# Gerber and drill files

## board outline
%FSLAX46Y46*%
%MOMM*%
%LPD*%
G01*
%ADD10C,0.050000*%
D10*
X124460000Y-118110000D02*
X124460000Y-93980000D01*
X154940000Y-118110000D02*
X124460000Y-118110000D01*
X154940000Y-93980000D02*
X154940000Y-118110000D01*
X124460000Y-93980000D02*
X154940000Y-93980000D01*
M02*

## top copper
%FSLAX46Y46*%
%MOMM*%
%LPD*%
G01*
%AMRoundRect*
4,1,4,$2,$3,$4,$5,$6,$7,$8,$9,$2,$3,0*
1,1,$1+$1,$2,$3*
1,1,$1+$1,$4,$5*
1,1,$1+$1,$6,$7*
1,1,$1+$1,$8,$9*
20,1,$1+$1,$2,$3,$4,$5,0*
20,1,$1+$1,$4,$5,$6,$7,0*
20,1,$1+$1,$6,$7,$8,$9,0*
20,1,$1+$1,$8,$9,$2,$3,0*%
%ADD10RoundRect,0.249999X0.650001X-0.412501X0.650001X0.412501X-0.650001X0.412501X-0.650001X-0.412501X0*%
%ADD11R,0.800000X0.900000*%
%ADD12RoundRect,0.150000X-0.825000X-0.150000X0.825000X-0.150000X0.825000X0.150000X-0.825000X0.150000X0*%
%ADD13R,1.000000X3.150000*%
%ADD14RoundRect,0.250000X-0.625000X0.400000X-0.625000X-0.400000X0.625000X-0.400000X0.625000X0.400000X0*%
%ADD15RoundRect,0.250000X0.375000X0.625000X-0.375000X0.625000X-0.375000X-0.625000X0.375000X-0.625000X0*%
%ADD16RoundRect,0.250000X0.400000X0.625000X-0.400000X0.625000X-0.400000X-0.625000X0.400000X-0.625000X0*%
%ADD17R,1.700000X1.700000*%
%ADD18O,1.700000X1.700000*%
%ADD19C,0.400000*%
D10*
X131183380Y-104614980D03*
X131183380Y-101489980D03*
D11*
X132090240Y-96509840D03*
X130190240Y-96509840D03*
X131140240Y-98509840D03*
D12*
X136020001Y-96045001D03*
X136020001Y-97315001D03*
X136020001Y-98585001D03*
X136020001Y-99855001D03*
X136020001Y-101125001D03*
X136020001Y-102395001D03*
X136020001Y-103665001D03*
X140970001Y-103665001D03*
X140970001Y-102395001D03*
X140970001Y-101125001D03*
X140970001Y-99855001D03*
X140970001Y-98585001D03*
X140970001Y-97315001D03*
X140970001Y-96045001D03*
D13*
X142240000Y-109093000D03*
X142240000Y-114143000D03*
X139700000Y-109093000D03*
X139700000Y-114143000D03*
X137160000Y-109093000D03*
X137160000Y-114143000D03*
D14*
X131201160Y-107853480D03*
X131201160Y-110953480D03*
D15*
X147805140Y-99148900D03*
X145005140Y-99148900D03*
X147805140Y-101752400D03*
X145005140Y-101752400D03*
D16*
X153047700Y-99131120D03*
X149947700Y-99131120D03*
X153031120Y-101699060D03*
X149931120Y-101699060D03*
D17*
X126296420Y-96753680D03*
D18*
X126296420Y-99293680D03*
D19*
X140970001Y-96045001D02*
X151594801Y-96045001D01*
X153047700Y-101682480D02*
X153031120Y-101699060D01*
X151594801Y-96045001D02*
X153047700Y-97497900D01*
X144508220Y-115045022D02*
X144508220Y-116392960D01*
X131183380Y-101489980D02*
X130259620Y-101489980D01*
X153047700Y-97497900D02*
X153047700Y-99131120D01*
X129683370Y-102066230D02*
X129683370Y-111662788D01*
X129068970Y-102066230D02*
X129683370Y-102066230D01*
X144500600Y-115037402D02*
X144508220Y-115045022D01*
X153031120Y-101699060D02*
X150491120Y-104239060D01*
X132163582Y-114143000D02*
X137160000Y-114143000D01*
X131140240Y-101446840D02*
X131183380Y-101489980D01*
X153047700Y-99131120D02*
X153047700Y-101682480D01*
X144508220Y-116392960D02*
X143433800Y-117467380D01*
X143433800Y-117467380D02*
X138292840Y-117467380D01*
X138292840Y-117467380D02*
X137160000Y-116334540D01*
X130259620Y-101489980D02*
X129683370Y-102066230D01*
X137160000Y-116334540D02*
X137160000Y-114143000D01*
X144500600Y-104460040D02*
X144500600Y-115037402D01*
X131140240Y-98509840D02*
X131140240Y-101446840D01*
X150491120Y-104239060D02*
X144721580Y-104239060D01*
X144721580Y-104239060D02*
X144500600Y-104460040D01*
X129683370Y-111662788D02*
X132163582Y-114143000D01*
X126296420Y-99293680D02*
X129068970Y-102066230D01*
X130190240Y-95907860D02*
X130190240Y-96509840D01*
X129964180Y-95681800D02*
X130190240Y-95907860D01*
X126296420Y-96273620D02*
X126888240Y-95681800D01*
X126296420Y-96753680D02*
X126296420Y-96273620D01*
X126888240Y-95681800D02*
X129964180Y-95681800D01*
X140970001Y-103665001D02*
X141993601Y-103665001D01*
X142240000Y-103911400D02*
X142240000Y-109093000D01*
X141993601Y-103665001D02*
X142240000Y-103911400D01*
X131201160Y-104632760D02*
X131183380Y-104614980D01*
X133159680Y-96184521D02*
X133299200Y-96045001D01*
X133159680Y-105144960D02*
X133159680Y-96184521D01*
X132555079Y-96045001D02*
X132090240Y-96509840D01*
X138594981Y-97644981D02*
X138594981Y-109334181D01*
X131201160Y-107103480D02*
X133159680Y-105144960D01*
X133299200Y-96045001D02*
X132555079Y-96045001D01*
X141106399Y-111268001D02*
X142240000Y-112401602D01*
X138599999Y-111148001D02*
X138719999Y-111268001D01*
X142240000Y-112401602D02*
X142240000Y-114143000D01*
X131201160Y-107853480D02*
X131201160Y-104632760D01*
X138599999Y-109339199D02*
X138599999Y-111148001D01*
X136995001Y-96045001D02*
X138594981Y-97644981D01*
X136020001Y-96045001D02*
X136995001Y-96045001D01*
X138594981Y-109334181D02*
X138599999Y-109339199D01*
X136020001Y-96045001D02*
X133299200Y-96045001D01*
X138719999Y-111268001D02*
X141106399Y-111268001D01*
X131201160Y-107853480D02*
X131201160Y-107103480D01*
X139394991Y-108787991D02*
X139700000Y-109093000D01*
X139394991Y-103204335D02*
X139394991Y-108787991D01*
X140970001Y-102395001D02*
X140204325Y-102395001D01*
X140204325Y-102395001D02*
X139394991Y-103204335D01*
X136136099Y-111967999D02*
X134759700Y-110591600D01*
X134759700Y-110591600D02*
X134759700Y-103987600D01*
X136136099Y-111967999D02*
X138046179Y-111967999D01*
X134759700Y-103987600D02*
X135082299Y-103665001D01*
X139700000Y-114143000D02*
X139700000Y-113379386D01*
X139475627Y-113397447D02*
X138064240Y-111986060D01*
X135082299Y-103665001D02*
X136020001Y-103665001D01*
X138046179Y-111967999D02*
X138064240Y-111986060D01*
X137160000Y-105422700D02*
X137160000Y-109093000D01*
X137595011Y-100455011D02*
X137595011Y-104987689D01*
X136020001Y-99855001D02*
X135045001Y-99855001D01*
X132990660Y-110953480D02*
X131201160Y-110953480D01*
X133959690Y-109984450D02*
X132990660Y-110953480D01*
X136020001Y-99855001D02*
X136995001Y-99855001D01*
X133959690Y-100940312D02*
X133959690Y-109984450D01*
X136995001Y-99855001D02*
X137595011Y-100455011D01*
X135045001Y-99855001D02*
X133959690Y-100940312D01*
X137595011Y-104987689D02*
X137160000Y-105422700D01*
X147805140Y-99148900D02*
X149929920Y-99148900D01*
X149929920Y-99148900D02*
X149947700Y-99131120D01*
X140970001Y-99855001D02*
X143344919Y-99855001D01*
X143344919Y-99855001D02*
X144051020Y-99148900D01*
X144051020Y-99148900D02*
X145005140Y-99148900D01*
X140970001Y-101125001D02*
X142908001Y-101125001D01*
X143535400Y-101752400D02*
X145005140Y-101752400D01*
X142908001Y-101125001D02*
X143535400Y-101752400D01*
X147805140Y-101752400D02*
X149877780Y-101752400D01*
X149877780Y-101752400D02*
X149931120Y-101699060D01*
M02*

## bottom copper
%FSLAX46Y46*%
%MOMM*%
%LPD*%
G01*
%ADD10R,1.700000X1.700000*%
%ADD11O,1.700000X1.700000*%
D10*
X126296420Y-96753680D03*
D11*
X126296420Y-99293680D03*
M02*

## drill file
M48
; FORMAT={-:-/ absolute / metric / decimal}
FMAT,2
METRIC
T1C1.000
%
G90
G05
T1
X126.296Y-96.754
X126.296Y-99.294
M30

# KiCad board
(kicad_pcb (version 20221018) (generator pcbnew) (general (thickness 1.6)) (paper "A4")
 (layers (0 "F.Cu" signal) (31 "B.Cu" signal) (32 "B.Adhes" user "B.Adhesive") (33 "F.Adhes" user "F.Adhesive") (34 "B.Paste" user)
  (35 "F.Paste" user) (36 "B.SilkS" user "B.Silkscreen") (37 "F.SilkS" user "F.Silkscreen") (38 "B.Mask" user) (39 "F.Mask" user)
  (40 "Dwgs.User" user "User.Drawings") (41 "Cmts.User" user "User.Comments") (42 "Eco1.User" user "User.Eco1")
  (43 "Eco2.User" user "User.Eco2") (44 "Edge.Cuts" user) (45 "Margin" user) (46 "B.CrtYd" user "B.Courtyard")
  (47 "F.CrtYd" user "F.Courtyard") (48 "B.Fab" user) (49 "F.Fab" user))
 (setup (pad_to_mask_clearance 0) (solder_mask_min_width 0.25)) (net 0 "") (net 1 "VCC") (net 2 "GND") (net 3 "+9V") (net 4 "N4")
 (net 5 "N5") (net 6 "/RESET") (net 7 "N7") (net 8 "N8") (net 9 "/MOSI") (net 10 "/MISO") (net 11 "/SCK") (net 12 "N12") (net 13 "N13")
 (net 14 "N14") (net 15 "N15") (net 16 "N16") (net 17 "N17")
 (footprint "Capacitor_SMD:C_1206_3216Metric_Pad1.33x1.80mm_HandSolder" (layer "F.Cu") (at 131.18338 103.05248 90)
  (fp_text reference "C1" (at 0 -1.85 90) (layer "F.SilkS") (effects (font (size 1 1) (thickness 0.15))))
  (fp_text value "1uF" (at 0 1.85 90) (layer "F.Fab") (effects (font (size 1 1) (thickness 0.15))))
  (pad "1" smd roundrect (at -1.5625 0 90) (size 1.325 1.8) (layers "F.Cu" "F.Paste" "F.Mask") (roundrect_rratio 0.1886784906) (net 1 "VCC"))
  (pad "2" smd roundrect (at 1.5625 0 90) (size 1.325 1.8) (layers "F.Cu" "F.Paste" "F.Mask") (roundrect_rratio 0.1886784906) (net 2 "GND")))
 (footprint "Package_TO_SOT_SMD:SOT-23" (layer "F.Cu") (at 131.14024 97.50984 -90)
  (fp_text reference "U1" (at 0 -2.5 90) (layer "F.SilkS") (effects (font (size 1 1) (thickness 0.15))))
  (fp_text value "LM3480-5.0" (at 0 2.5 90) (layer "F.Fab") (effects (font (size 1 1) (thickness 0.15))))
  (pad "1" smd rect (at -1 -0.95 270) (size 0.9 0.8) (layers "F.Cu" "F.Paste" "F.Mask") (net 1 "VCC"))
  (pad "2" smd rect (at -1 0.95 270) (size 0.9 0.8) (layers "F.Cu" "F.Paste" "F.Mask") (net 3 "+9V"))
  (pad "3" smd rect (at 1 0 270) (size 0.9 0.8) (layers "F.Cu" "F.Paste" "F.Mask") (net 2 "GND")))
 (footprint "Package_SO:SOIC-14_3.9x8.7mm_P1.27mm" (layer "F.Cu") (at 138.495001 99.855001)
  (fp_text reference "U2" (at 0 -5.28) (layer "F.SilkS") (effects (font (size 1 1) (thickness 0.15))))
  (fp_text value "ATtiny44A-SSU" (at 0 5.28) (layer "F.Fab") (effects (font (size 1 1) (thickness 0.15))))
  (pad "1" smd roundrect (at -2.475 -3.81) (size 1.95 0.6) (layers "F.Cu" "F.Paste" "F.Mask") (roundrect_rratio 0.25) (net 1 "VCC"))
  (pad "2" smd roundrect (at -2.475 -2.54) (size 1.95 0.6) (layers "F.Cu" "F.Paste" "F.Mask") (roundrect_rratio 0.25) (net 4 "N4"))
  (pad "3" smd roundrect (at -2.475 -1.27) (size 1.95 0.6) (layers "F.Cu" "F.Paste" "F.Mask") (roundrect_rratio 0.25) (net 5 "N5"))
  (pad "4" smd roundrect (at -2.475 0) (size 1.95 0.6) (layers "F.Cu" "F.Paste" "F.Mask") (roundrect_rratio 0.25) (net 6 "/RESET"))
  (pad "5" smd roundrect (at -2.475 1.27) (size 1.95 0.6) (layers "F.Cu" "F.Paste" "F.Mask") (roundrect_rratio 0.25) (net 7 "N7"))
  (pad "6" smd roundrect (at -2.475 2.54) (size 1.95 0.6) (layers "F.Cu" "F.Paste" "F.Mask") (roundrect_rratio 0.25) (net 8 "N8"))
  (pad "7" smd roundrect (at -2.475 3.81) (size 1.95 0.6) (layers "F.Cu" "F.Paste" "F.Mask") (roundrect_rratio 0.25) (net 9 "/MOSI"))
  (pad "8" smd roundrect (at 2.475 3.81) (size 1.95 0.6) (layers "F.Cu" "F.Paste" "F.Mask") (roundrect_rratio 0.25) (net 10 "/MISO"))
  (pad "9" smd roundrect (at 2.475 2.54) (size 1.95 0.6) (layers "F.Cu" "F.Paste" "F.Mask") (roundrect_rratio 0.25) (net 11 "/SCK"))
  (pad "10" smd roundrect (at 2.475 1.27) (size 1.95 0.6) (layers "F.Cu" "F.Paste" "F.Mask") (roundrect_rratio 0.25) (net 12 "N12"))
  (pad "11" smd roundrect (at 2.475 0) (size 1.95 0.6) (layers "F.Cu" "F.Paste" "F.Mask") (roundrect_rratio 0.25) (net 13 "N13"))
  (pad "12" smd roundrect (at 2.475 -1.27) (size 1.95 0.6) (layers "F.Cu" "F.Paste" "F.Mask") (roundrect_rratio 0.25) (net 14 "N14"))
  (pad "13" smd roundrect (at 2.475 -2.54) (size 1.95 0.6) (layers "F.Cu" "F.Paste" "F.Mask") (roundrect_rratio 0.25) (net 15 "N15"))
  (pad "14" smd roundrect (at 2.475 -3.81) (size 1.95 0.6) (layers "F.Cu" "F.Paste" "F.Mask") (roundrect_rratio 0.25) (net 2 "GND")))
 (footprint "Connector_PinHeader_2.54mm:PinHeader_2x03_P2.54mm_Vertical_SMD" (layer "F.Cu") (at 139.7 111.618 -90)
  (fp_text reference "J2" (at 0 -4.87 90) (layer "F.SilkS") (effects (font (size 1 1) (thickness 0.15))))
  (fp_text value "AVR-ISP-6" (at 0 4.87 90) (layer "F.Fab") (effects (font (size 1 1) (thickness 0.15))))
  (pad "1" smd rect (at -2.525 -2.54 270) (size 3.15 1) (layers "F.Cu" "F.Paste" "F.Mask") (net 10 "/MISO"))
  (pad "2" smd rect (at 2.525 -2.54 270) (size 3.15 1) (layers "F.Cu" "F.Paste" "F.Mask") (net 1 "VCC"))
  (pad "3" smd rect (at -2.525 0 270) (size 3.15 1) (layers "F.Cu" "F.Paste" "F.Mask") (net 11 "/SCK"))
  (pad "4" smd rect (at 2.525 0 270) (size 3.15 1) (layers "F.Cu" "F.Paste" "F.Mask") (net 9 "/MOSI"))
  (pad "5" smd rect (at -2.525 2.54 270) (size 3.15 1) (layers "F.Cu" "F.Paste" "F.Mask") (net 6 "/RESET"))
  (pad "6" smd rect (at 2.525 2.54 270) (size 3.15 1) (layers "F.Cu" "F.Paste" "F.Mask") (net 2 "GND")))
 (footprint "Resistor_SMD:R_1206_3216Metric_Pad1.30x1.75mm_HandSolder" (layer "F.Cu") (at 131.20116 109.40348 -90)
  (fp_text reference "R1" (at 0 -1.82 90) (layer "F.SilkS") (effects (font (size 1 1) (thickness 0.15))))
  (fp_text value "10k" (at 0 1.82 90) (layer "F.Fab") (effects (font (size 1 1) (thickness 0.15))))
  (pad "1" smd roundrect (at -1.55 0 270) (size 1.3 1.75) (layers "F.Cu" "F.Paste" "F.Mask") (roundrect_rratio 0.1923076923) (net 1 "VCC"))
  (pad "2" smd roundrect (at 1.55 0 270) (size 1.3 1.75) (layers "F.Cu" "F.Paste" "F.Mask") (roundrect_rratio 0.1923076923) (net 6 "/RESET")))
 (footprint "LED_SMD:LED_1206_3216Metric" (layer "F.Cu") (at 146.40514 99.1489 180)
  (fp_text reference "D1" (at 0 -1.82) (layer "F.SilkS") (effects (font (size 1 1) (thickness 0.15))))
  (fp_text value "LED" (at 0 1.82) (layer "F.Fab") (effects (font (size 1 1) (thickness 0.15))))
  (pad "1" smd roundrect (at -1.4 0 180) (size 1.25 1.75) (layers "F.Cu" "F.Paste" "F.Mask") (roundrect_rratio 0.2) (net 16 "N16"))
  (pad "2" smd roundrect (at 1.4 0 180) (size 1.25 1.75) (layers "F.Cu" "F.Paste" "F.Mask") (roundrect_rratio 0.2) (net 13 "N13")))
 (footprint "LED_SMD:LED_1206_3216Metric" (layer "F.Cu") (at 146.40514 101.7524 180)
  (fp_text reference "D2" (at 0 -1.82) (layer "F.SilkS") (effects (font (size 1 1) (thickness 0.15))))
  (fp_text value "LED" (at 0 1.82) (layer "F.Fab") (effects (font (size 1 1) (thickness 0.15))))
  (pad "1" smd roundrect (at -1.4 0 180) (size 1.25 1.75) (layers "F.Cu" "F.Paste" "F.Mask") (roundrect_rratio 0.2) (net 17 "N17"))
  (pad "2" smd roundrect (at 1.4 0 180) (size 1.25 1.75) (layers "F.Cu" "F.Paste" "F.Mask") (roundrect_rratio 0.2) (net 12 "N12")))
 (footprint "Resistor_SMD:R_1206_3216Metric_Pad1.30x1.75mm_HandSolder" (layer "F.Cu") (at 151.4977 99.13112 180)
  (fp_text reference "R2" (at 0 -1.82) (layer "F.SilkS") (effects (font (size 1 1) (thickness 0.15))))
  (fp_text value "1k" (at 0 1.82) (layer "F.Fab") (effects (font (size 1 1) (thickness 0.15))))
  (pad "1" smd roundrect (at -1.55 0 180) (size 1.3 1.75) (layers "F.Cu" "F.Paste" "F.Mask") (roundrect_rratio 0.1923076923) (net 2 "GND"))
  (pad "2" smd roundrect (at 1.55 0 180) (size 1.3 1.75) (layers "F.Cu" "F.Paste" "F.Mask") (roundrect_rratio 0.1923076923) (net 16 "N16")))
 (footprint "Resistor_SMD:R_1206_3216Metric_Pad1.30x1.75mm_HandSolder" (layer "F.Cu") (at 151.48112 101.69906 180)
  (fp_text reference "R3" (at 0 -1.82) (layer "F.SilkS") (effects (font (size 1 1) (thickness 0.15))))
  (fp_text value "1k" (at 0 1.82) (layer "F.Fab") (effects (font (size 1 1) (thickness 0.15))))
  (pad "1" smd roundrect (at -1.55 0 180) (size 1.3 1.75) (layers "F.Cu" "F.Paste" "F.Mask") (roundrect_rratio 0.1923076923) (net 2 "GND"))
  (pad "2" smd roundrect (at 1.55 0 180) (size 1.3 1.75) (layers "F.Cu" "F.Paste" "F.Mask") (roundrect_rratio 0.1923076923) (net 17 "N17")))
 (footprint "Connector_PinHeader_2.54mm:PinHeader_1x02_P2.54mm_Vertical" (layer "F.Cu") (at 126.29642 96.75368)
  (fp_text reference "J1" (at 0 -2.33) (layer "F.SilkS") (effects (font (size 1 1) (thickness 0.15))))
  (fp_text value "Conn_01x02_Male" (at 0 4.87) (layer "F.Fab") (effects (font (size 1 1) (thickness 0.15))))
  (pad "1" thru_hole rect (at 0 0) (size 1.7 1.7) (drill 1) (layers "*.Cu" "*.Mask") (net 3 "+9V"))
  (pad "2" thru_hole oval (at 0 2.54) (size 1.7 1.7) (drill 1) (layers "*.Cu" "*.Mask") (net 2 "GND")))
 (gr_line (start 124.46 118.11) (end 124.46 93.98) (stroke (width 0.05) (type solid)) (layer "Edge.Cuts"))
 (gr_line (start 154.94 118.11) (end 124.46 118.11) (stroke (width 0.05) (type solid)) (layer "Edge.Cuts"))
 (gr_line (start 154.94 93.98) (end 154.94 118.11) (stroke (width 0.05) (type solid)) (layer "Edge.Cuts"))
 (gr_line (start 124.46 93.98) (end 154.94 93.98) (stroke (width 0.05) (type solid)) (layer "Edge.Cuts"))
 (segment (start 140.970001 96.045001) (end 151.594801 96.045001) (width 0.4) (layer "F.Cu") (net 2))
 (segment (start 153.0477 101.68248) (end 153.03112 101.69906) (width 0.4) (layer "F.Cu") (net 2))
 (segment (start 151.594801 96.045001) (end 153.0477 97.4979) (width 0.4) (layer "F.Cu") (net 2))
 (segment (start 144.50822 115.045022) (end 144.50822 116.39296) (width 0.4) (layer "F.Cu") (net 2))
 (segment (start 131.18338 101.48998) (end 130.25962 101.48998) (width 0.4) (layer "F.Cu") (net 2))
 (segment (start 153.0477 97.4979) (end 153.0477 99.13112) (width 0.4) (layer "F.Cu") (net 2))
 (segment (start 129.68337 102.06623) (end 129.68337 111.662788) (width 0.4) (layer "F.Cu") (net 2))
 (segment (start 129.06897 102.06623) (end 129.68337 102.06623) (width 0.4) (layer "F.Cu") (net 2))
 (segment (start 144.5006 115.037402) (end 144.50822 115.045022) (width 0.4) (layer "F.Cu") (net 2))
 (segment (start 153.03112 101.69906) (end 150.49112 104.23906) (width 0.4) (layer "F.Cu") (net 2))
 (segment (start 132.163582 114.143) (end 137.16 114.143) (width 0.4) (layer "F.Cu") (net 2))
 (segment (start 131.14024 101.44684) (end 131.18338 101.48998) (width 0.4) (layer "F.Cu") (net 2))
 (segment (start 153.0477 99.13112) (end 153.0477 101.68248) (width 0.4) (layer "F.Cu") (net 2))
 (segment (start 144.50822 116.39296) (end 143.4338 117.46738) (width 0.4) (layer "F.Cu") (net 2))
 (segment (start 143.4338 117.46738) (end 138.29284 117.46738) (width 0.4) (layer "F.Cu") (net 2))
 (segment (start 138.29284 117.46738) (end 137.16 116.33454) (width 0.4) (layer "F.Cu") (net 2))
 (segment (start 130.25962 101.48998) (end 129.68337 102.06623) (width 0.4) (layer "F.Cu") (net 2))
 (segment (start 137.16 116.33454) (end 137.16 114.143) (width 0.4) (layer "F.Cu") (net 2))
 (segment (start 144.5006 104.46004) (end 144.5006 115.037402) (width 0.4) (layer "F.Cu") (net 2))
 (segment (start 131.14024 98.50984) (end 131.14024 101.44684) (width 0.4) (layer "F.Cu") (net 2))
 (segment (start 150.49112 104.23906) (end 144.72158 104.23906) (width 0.4) (layer "F.Cu") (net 2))
 (segment (start 144.72158 104.23906) (end 144.5006 104.46004) (width 0.4) (layer "F.Cu") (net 2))
 (segment (start 129.68337 111.662788) (end 132.163582 114.143) (width 0.4) (layer "F.Cu") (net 2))
 (segment (start 126.29642 99.29368) (end 129.06897 102.06623) (width 0.4) (layer "F.Cu") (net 2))
 (segment (start 130.19024 95.90786) (end 130.19024 96.50984) (width 0.4) (layer "F.Cu") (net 3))
 (segment (start 129.96418 95.6818) (end 130.19024 95.90786) (width 0.4) (layer "F.Cu") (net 3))
 (segment (start 126.29642 96.27362) (end 126.88824 95.6818) (width 0.4) (layer "F.Cu") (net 3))
 (segment (start 126.29642 96.75368) (end 126.29642 96.27362) (width 0.4) (layer "F.Cu") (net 3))
 (segment (start 126.88824 95.6818) (end 129.96418 95.6818) (width 0.4) (layer "F.Cu") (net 3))
 (segment (start 140.970001 103.665001) (end 141.993601 103.665001) (width 0.4) (layer "F.Cu") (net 10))
 (segment (start 142.24 103.9114) (end 142.24 109.093) (width 0.4) (layer "F.Cu") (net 10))
 (segment (start 141.993601 103.665001) (end 142.24 103.9114) (width 0.4) (layer "F.Cu") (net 10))
 (segment (start 131.20116 104.63276) (end 131.18338 104.61498) (width 0.4) (layer "F.Cu") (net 1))
 (segment (start 133.15968 96.184521) (end 133.2992 96.045001) (width 0.4) (layer "F.Cu") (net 1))
 (segment (start 133.15968 105.14496) (end 133.15968 96.184521) (width 0.4) (layer "F.Cu") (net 1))
 (segment (start 132.555079 96.045001) (end 132.09024 96.50984) (width 0.4) (layer "F.Cu") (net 1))
 (segment (start 138.594981 97.644981) (end 138.594981 109.334181) (width 0.4) (layer "F.Cu") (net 1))
 (segment (start 131.20116 107.10348) (end 133.15968 105.14496) (width 0.4) (layer "F.Cu") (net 1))
 (segment (start 133.2992 96.045001) (end 132.555079 96.045001) (width 0.4) (layer "F.Cu") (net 1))
 (segment (start 141.106399 111.268001) (end 142.24 112.401602) (width 0.4) (layer "F.Cu") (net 1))
 (segment (start 138.599999 111.148001) (end 138.719999 111.268001) (width 0.4) (layer "F.Cu") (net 1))
 (segment (start 142.24 112.401602) (end 142.24 114.143) (width 0.4) (layer "F.Cu") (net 1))
 (segment (start 131.20116 107.85348) (end 131.20116 104.63276) (width 0.4) (layer "F.Cu") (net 1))
 (segment (start 138.599999 109.339199) (end 138.599999 111.148001) (width 0.4) (layer "F.Cu") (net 1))
 (segment (start 136.995001 96.045001) (end 138.594981 97.644981) (width 0.4) (layer "F.Cu") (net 1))
 (segment (start 136.020001 96.045001) (end 136.995001 96.045001) (width 0.4) (layer "F.Cu") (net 1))
 (segment (start 138.594981 109.334181) (end 138.599999 109.339199) (width 0.4) (layer "F.Cu") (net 1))
 (segment (start 136.020001 96.045001) (end 133.2992 96.045001) (width 0.4) (layer "F.Cu") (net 1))
 (segment (start 138.719999 111.268001) (end 141.106399 111.268001) (width 0.4) (layer "F.Cu") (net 1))
 (segment (start 131.20116 107.85348) (end 131.20116 107.10348) (width 0.4) (layer "F.Cu") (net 1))
 (segment (start 139.394991 108.787991) (end 139.7 109.093) (width 0.4) (layer "F.Cu") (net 11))
 (segment (start 139.394991 103.204335) (end 139.394991 108.787991) (width 0.4) (layer "F.Cu") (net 11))
 (segment (start 140.970001 102.395001) (end 140.204325 102.395001) (width 0.4) (layer "F.Cu") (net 11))
 (segment (start 140.204325 102.395001) (end 139.394991 103.204335) (width 0.4) (layer "F.Cu") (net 11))
 (segment (start 136.136099 111.967999) (end 134.7597 110.5916) (width 0.4) (layer "F.Cu") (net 9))
 (segment (start 134.7597 110.5916) (end 134.7597 103.9876) (width 0.4) (layer "F.Cu") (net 9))
 (segment (start 136.136099 111.967999) (end 138.046179 111.967999) (width 0.4) (layer "F.Cu") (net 9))
 (segment (start 134.7597 103.9876) (end 135.082299 103.665001) (width 0.4) (layer "F.Cu") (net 9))
 (segment (start 139.7 114.143) (end 139.7 113.379386) (width 0.4) (layer "F.Cu") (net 9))
 (segment (start 139.475627 113.397447) (end 138.06424 111.98606) (width 0.4) (layer "F.Cu") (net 9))
 (segment (start 135.082299 103.665001) (end 136.020001 103.665001) (width 0.4) (layer "F.Cu") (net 9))
 (segment (start 138.046179 111.967999) (end 138.06424 111.98606) (width 0.4) (layer "F.Cu") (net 9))
 (segment (start 137.16 105.4227) (end 137.16 109.093) (width 0.4) (layer "F.Cu") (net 6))
 (segment (start 137.595011 100.455011) (end 137.595011 104.987689) (width 0.4) (layer "F.Cu") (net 6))
 (segment (start 136.020001 99.855001) (end 135.045001 99.855001) (width 0.4) (layer "F.Cu") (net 6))
 (segment (start 132.99066 110.95348) (end 131.20116 110.95348) (width 0.4) (layer "F.Cu") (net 6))
 (segment (start 133.95969 109.98445) (end 132.99066 110.95348) (width 0.4) (layer "F.Cu") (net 6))
 (segment (start 136.020001 99.855001) (end 136.995001 99.855001) (width 0.4) (layer "F.Cu") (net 6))
 (segment (start 133.95969 100.940312) (end 133.95969 109.98445) (width 0.4) (layer "F.Cu") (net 6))
 (segment (start 136.995001 99.855001) (end 137.595011 100.455011) (width 0.4) (layer "F.Cu") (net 6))
 (segment (start 135.045001 99.855001) (end 133.95969 100.940312) (width 0.4) (layer "F.Cu") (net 6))
 (segment (start 137.595011 104.987689) (end 137.16 105.4227) (width 0.4) (layer "F.Cu") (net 6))
 (segment (start 147.80514 99.1489) (end 149.92992 99.1489) (width 0.4) (layer "F.Cu") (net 16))
 (segment (start 149.92992 99.1489) (end 149.9477 99.13112) (width 0.4) (layer "F.Cu") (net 16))
 (segment (start 140.970001 99.855001) (end 143.344919 99.855001) (width 0.4) (layer "F.Cu") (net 13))
 (segment (start 143.344919 99.855001) (end 144.05102 99.1489) (width 0.4) (layer "F.Cu") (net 13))
 (segment (start 144.05102 99.1489) (end 145.00514 99.1489) (width 0.4) (layer "F.Cu") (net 13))
 (segment (start 140.970001 101.125001) (end 142.908001 101.125001) (width 0.4) (layer "F.Cu") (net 12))
 (segment (start 143.5354 101.7524) (end 145.00514 101.7524) (width 0.4) (layer "F.Cu") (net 12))
 (segment (start 142.908001 101.125001) (end 143.5354 101.7524) (width 0.4) (layer "F.Cu") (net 12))
 (segment (start 147.80514 101.7524) (end 149.87778 101.7524) (width 0.4) (layer "F.Cu") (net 17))
 (segment (start 149.87778 101.7524) (end 149.93112 101.69906) (width 0.4) (layer "F.Cu") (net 17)))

